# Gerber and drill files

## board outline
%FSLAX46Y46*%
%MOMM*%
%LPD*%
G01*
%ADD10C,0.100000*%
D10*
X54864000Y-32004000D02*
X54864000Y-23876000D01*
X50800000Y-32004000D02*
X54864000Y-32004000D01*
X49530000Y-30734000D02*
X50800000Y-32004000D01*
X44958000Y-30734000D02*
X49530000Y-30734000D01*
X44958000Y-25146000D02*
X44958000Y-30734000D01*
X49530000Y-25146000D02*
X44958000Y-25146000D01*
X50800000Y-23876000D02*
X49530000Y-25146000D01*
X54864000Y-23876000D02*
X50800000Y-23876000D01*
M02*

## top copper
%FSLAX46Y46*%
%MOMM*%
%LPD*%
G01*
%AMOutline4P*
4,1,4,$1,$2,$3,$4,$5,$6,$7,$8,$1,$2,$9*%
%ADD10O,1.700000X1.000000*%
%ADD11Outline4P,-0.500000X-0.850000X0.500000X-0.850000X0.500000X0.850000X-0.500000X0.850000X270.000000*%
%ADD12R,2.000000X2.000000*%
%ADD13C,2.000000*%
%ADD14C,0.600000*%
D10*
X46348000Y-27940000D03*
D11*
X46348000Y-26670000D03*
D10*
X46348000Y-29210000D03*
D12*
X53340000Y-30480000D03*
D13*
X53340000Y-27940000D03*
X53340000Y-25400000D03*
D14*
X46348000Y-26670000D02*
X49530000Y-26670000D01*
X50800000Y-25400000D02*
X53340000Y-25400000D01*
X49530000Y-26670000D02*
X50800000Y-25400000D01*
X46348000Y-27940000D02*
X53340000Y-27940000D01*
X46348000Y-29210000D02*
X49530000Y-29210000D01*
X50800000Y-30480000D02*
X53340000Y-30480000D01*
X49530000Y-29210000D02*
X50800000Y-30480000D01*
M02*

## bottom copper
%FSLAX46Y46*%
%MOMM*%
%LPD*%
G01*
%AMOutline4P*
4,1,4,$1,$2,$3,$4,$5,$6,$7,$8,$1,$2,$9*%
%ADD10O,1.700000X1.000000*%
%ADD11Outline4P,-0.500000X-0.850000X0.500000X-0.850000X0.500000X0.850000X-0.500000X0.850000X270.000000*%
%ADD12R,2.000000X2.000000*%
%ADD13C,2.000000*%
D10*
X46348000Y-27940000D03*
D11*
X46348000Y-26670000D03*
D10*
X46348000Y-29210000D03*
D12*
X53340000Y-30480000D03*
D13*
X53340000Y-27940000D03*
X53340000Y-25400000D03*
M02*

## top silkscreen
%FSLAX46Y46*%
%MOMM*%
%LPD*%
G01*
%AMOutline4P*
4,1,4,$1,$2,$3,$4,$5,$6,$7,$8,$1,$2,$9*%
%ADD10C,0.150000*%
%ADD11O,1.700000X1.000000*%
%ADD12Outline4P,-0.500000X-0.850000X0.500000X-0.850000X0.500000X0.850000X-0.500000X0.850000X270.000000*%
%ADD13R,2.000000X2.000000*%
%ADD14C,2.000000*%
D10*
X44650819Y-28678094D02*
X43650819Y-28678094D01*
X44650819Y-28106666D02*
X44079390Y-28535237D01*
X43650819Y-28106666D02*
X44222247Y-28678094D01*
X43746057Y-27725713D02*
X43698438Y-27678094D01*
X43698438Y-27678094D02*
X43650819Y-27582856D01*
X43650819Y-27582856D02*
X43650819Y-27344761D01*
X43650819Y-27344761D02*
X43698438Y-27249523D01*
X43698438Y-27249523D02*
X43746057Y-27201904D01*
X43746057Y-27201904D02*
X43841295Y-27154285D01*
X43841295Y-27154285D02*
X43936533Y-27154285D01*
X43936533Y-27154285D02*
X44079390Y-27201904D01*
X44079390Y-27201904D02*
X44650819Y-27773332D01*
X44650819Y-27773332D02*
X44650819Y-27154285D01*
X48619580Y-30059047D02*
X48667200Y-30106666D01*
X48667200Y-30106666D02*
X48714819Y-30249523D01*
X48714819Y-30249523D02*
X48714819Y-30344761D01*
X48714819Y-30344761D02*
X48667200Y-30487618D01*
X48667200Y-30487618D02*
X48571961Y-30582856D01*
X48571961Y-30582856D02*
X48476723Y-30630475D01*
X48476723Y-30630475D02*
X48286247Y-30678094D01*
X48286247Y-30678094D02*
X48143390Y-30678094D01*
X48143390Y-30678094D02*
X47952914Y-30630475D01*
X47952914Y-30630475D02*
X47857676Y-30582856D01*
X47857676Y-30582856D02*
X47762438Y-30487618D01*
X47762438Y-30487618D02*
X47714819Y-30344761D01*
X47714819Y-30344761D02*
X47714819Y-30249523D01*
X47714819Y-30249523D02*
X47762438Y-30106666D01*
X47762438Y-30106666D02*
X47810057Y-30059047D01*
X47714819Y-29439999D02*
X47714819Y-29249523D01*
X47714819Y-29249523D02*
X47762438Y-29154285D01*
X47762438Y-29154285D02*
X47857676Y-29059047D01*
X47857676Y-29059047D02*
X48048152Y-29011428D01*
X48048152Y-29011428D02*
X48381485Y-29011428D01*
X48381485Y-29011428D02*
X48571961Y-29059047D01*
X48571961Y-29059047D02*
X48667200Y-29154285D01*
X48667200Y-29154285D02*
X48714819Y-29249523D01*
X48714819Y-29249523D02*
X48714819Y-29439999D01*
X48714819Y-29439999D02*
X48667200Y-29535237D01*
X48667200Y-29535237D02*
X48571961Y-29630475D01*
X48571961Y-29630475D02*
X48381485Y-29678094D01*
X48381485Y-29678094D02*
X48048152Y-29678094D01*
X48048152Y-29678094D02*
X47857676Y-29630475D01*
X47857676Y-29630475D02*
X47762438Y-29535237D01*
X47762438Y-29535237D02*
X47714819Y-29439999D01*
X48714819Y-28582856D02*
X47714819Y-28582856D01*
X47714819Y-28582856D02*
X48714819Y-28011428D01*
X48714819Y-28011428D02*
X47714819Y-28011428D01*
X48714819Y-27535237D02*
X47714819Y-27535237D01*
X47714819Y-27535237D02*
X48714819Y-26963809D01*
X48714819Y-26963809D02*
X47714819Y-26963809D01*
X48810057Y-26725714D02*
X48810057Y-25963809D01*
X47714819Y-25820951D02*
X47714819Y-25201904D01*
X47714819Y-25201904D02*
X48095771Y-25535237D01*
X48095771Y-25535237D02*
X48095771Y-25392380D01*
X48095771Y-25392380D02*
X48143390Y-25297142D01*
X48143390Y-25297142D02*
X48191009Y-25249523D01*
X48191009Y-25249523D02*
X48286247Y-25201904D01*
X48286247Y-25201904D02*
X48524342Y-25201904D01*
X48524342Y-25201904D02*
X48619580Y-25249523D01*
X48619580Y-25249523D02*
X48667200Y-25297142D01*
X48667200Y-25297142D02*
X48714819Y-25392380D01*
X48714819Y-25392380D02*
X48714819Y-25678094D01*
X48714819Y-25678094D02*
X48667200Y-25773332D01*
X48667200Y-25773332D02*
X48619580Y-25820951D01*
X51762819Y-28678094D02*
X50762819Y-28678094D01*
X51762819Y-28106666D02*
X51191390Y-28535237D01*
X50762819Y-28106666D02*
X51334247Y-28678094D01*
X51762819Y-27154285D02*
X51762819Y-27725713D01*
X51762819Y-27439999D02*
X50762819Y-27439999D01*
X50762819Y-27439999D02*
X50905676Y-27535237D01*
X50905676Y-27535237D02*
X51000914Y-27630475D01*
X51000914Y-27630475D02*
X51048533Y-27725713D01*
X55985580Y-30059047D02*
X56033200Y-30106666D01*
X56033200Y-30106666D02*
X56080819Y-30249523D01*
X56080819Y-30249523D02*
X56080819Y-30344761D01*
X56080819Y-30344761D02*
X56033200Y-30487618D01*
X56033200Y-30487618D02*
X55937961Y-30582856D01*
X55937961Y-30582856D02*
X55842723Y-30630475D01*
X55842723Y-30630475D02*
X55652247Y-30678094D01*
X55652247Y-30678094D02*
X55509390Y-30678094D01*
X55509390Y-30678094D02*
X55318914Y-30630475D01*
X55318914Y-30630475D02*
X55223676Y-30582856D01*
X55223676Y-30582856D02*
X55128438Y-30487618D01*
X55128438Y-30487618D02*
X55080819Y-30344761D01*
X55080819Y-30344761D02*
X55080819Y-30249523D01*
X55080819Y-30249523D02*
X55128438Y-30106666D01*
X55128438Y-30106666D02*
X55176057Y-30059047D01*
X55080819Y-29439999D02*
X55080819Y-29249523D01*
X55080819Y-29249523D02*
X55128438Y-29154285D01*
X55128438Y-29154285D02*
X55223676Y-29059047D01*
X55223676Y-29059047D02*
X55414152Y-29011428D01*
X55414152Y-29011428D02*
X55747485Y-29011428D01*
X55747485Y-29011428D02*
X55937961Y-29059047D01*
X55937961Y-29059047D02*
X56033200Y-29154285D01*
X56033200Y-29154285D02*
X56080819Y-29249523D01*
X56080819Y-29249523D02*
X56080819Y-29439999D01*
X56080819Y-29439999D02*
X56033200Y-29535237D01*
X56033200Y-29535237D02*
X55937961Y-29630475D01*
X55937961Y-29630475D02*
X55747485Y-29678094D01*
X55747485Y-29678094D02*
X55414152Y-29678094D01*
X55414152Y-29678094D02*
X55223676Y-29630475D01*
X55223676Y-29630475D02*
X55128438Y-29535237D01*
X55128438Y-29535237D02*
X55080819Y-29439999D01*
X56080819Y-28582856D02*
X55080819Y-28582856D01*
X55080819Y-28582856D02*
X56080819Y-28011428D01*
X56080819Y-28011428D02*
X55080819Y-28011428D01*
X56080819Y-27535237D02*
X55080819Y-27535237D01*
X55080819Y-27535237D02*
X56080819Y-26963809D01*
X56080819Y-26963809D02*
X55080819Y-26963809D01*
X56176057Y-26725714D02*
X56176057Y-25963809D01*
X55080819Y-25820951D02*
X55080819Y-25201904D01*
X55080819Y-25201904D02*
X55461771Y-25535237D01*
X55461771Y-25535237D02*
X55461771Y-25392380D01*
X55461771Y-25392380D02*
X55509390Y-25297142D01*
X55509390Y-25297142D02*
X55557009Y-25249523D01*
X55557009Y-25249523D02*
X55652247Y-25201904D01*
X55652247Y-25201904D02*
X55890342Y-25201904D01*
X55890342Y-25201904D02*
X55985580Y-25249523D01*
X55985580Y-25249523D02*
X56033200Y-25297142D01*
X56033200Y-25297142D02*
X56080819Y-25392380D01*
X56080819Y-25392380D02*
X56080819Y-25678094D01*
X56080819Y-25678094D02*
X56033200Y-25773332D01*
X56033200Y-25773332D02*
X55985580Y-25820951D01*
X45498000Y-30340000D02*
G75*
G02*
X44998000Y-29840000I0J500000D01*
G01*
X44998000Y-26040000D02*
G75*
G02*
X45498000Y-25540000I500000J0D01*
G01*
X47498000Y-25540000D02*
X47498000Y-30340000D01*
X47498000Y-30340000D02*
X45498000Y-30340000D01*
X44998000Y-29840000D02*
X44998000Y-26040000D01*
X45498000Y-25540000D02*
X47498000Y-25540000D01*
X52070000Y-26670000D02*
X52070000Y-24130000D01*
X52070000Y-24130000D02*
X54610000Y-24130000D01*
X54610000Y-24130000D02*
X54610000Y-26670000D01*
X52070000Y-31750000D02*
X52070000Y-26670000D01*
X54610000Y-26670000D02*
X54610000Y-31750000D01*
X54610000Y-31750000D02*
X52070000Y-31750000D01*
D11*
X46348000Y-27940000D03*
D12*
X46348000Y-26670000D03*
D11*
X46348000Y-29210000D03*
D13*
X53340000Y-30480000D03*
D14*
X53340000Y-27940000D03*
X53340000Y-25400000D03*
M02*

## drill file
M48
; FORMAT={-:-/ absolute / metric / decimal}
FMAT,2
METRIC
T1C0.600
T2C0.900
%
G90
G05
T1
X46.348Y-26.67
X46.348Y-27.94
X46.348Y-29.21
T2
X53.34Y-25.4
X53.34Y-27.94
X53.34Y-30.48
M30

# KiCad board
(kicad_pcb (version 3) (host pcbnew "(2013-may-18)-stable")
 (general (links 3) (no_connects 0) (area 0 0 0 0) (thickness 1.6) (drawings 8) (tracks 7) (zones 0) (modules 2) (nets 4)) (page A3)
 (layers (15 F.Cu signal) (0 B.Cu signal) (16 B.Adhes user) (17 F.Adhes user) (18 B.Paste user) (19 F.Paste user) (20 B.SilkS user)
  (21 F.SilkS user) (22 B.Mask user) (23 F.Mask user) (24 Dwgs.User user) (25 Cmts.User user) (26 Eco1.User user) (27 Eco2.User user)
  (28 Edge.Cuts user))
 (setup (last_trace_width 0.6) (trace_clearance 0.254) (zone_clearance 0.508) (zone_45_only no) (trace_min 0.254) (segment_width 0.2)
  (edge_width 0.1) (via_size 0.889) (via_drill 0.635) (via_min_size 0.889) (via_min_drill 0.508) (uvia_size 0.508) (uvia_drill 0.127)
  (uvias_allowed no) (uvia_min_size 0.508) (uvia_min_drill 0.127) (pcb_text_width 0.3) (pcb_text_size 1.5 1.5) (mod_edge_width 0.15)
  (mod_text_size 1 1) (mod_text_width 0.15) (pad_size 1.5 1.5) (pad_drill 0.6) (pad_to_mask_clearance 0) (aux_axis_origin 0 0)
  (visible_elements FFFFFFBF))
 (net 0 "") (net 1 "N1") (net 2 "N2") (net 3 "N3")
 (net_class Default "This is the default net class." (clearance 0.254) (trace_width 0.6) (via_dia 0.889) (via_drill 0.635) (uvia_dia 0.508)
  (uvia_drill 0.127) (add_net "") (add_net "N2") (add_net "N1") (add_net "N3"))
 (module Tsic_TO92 (layer F.Cu) (at 48.26 27.94 270)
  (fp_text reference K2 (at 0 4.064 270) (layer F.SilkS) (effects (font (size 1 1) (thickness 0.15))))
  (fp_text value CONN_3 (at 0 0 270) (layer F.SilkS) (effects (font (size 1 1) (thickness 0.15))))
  (fp_arc (start 1.9 2.762) (end 2.4 2.762) (angle 90) (layer F.SilkS) (width 0.15))
  (fp_arc (start -1.9 2.762) (end -1.9 3.262) (angle 90) (layer F.SilkS) (width 0.15))
  (fp_line (start -2.4 0.762) (end 2.4 0.762) (layer F.SilkS) (width 0.15))
  (fp_line (start 2.4 0.762) (end 2.4 2.762) (layer F.SilkS) (width 0.15))
  (fp_line (start 1.9 3.262) (end -1.9 3.262) (layer F.SilkS) (width 0.15))
  (fp_line (start -2.4 2.762) (end -2.4 0.762) (layer F.SilkS) (width 0.15))
  (pad 2 thru_hole oval (at 0 1.912 270) (size 1 1.7) (drill 0.6) (layers *.Cu *.Mask F.SilkS) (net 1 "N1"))
  (pad 1 thru_hole trapezoid (at -1.27 1.912 270) (size 1 1.7) (drill 0.6) (layers *.Cu *.Mask F.SilkS) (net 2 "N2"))
  (pad 3 thru_hole oval (at 1.27 1.912 270) (size 1 1.7) (drill 0.6) (layers *.Cu *.Mask F.SilkS) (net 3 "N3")))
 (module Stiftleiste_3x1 (layer F.Cu) (at 53.34 27.94 90)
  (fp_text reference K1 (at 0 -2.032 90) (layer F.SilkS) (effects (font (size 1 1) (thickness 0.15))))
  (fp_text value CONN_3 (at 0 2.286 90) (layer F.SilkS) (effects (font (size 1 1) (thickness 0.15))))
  (fp_line (start 1.27 -1.27) (end 3.81 -1.27) (layer F.SilkS) (width 0.15))
  (fp_line (start 3.81 -1.27) (end 3.81 1.27) (layer F.SilkS) (width 0.15))
  (fp_line (start 3.81 1.27) (end 1.27 1.27) (layer F.SilkS) (width 0.15))
  (fp_line (start -3.81 -1.27) (end 1.27 -1.27) (layer F.SilkS) (width 0.15))
  (fp_line (start 1.27 1.27) (end -3.81 1.27) (layer F.SilkS) (width 0.15))
  (fp_line (start -3.81 1.27) (end -3.81 -1.27) (layer F.SilkS) (width 0.15))
  (pad 1 thru_hole rect (at -2.54 0 90) (size 2 2) (drill 0.9) (layers *.Cu *.Mask F.SilkS) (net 3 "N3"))
  (pad 2 thru_hole circle (at 0 0 90) (size 2 2) (drill 0.9) (layers *.Cu *.Mask F.SilkS) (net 1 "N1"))
  (pad 3 thru_hole circle (at 2.54 0 90) (size 2 2) (drill 0.9) (layers *.Cu *.Mask F.SilkS) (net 2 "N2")))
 (gr_line (start 54.864 32.004) (end 54.864 23.876) (angle 90) (layer Edge.Cuts) (width 0.1))
 (gr_line (start 50.8 32.004) (end 54.864 32.004) (angle 90) (layer Edge.Cuts) (width 0.1))
 (gr_line (start 49.53 30.734) (end 50.8 32.004) (angle 90) (layer Edge.Cuts) (width 0.1))
 (gr_line (start 44.958 30.734) (end 49.53 30.734) (angle 90) (layer Edge.Cuts) (width 0.1))
 (gr_line (start 44.958 25.146) (end 44.958 30.734) (angle 90) (layer Edge.Cuts) (width 0.1))
 (gr_line (start 49.53 25.146) (end 44.958 25.146) (angle 90) (layer Edge.Cuts) (width 0.1))
 (gr_line (start 50.8 23.876) (end 49.53 25.146) (angle 90) (layer Edge.Cuts) (width 0.1))
 (gr_line (start 54.864 23.876) (end 50.8 23.876) (angle 90) (layer Edge.Cuts) (width 0.1))
 (segment (start 46.348 26.67) (end 49.53 26.67) (width 0.6) (layer F.Cu) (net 2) (status 400000))
 (segment (start 50.8 25.4) (end 53.34 25.4) (width 0.6) (layer F.Cu) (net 2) (status 800000))
 (segment (start 49.53 26.67) (end 50.8 25.4) (width 0.6) (layer F.Cu) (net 2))
 (segment (start 46.348 27.94) (end 53.34 27.94) (width 0.6) (layer F.Cu) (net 1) (status C00000))
 (segment (start 46.348 29.21) (end 49.53 29.21) (width 0.6) (layer F.Cu) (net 3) (status 400000))
 (segment (start 50.8 30.48) (end 53.34 30.48) (width 0.6) (layer F.Cu) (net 3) (status 800000))
 (segment (start 49.53 29.21) (end 50.8 30.48) (width 0.6) (layer F.Cu) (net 3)))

